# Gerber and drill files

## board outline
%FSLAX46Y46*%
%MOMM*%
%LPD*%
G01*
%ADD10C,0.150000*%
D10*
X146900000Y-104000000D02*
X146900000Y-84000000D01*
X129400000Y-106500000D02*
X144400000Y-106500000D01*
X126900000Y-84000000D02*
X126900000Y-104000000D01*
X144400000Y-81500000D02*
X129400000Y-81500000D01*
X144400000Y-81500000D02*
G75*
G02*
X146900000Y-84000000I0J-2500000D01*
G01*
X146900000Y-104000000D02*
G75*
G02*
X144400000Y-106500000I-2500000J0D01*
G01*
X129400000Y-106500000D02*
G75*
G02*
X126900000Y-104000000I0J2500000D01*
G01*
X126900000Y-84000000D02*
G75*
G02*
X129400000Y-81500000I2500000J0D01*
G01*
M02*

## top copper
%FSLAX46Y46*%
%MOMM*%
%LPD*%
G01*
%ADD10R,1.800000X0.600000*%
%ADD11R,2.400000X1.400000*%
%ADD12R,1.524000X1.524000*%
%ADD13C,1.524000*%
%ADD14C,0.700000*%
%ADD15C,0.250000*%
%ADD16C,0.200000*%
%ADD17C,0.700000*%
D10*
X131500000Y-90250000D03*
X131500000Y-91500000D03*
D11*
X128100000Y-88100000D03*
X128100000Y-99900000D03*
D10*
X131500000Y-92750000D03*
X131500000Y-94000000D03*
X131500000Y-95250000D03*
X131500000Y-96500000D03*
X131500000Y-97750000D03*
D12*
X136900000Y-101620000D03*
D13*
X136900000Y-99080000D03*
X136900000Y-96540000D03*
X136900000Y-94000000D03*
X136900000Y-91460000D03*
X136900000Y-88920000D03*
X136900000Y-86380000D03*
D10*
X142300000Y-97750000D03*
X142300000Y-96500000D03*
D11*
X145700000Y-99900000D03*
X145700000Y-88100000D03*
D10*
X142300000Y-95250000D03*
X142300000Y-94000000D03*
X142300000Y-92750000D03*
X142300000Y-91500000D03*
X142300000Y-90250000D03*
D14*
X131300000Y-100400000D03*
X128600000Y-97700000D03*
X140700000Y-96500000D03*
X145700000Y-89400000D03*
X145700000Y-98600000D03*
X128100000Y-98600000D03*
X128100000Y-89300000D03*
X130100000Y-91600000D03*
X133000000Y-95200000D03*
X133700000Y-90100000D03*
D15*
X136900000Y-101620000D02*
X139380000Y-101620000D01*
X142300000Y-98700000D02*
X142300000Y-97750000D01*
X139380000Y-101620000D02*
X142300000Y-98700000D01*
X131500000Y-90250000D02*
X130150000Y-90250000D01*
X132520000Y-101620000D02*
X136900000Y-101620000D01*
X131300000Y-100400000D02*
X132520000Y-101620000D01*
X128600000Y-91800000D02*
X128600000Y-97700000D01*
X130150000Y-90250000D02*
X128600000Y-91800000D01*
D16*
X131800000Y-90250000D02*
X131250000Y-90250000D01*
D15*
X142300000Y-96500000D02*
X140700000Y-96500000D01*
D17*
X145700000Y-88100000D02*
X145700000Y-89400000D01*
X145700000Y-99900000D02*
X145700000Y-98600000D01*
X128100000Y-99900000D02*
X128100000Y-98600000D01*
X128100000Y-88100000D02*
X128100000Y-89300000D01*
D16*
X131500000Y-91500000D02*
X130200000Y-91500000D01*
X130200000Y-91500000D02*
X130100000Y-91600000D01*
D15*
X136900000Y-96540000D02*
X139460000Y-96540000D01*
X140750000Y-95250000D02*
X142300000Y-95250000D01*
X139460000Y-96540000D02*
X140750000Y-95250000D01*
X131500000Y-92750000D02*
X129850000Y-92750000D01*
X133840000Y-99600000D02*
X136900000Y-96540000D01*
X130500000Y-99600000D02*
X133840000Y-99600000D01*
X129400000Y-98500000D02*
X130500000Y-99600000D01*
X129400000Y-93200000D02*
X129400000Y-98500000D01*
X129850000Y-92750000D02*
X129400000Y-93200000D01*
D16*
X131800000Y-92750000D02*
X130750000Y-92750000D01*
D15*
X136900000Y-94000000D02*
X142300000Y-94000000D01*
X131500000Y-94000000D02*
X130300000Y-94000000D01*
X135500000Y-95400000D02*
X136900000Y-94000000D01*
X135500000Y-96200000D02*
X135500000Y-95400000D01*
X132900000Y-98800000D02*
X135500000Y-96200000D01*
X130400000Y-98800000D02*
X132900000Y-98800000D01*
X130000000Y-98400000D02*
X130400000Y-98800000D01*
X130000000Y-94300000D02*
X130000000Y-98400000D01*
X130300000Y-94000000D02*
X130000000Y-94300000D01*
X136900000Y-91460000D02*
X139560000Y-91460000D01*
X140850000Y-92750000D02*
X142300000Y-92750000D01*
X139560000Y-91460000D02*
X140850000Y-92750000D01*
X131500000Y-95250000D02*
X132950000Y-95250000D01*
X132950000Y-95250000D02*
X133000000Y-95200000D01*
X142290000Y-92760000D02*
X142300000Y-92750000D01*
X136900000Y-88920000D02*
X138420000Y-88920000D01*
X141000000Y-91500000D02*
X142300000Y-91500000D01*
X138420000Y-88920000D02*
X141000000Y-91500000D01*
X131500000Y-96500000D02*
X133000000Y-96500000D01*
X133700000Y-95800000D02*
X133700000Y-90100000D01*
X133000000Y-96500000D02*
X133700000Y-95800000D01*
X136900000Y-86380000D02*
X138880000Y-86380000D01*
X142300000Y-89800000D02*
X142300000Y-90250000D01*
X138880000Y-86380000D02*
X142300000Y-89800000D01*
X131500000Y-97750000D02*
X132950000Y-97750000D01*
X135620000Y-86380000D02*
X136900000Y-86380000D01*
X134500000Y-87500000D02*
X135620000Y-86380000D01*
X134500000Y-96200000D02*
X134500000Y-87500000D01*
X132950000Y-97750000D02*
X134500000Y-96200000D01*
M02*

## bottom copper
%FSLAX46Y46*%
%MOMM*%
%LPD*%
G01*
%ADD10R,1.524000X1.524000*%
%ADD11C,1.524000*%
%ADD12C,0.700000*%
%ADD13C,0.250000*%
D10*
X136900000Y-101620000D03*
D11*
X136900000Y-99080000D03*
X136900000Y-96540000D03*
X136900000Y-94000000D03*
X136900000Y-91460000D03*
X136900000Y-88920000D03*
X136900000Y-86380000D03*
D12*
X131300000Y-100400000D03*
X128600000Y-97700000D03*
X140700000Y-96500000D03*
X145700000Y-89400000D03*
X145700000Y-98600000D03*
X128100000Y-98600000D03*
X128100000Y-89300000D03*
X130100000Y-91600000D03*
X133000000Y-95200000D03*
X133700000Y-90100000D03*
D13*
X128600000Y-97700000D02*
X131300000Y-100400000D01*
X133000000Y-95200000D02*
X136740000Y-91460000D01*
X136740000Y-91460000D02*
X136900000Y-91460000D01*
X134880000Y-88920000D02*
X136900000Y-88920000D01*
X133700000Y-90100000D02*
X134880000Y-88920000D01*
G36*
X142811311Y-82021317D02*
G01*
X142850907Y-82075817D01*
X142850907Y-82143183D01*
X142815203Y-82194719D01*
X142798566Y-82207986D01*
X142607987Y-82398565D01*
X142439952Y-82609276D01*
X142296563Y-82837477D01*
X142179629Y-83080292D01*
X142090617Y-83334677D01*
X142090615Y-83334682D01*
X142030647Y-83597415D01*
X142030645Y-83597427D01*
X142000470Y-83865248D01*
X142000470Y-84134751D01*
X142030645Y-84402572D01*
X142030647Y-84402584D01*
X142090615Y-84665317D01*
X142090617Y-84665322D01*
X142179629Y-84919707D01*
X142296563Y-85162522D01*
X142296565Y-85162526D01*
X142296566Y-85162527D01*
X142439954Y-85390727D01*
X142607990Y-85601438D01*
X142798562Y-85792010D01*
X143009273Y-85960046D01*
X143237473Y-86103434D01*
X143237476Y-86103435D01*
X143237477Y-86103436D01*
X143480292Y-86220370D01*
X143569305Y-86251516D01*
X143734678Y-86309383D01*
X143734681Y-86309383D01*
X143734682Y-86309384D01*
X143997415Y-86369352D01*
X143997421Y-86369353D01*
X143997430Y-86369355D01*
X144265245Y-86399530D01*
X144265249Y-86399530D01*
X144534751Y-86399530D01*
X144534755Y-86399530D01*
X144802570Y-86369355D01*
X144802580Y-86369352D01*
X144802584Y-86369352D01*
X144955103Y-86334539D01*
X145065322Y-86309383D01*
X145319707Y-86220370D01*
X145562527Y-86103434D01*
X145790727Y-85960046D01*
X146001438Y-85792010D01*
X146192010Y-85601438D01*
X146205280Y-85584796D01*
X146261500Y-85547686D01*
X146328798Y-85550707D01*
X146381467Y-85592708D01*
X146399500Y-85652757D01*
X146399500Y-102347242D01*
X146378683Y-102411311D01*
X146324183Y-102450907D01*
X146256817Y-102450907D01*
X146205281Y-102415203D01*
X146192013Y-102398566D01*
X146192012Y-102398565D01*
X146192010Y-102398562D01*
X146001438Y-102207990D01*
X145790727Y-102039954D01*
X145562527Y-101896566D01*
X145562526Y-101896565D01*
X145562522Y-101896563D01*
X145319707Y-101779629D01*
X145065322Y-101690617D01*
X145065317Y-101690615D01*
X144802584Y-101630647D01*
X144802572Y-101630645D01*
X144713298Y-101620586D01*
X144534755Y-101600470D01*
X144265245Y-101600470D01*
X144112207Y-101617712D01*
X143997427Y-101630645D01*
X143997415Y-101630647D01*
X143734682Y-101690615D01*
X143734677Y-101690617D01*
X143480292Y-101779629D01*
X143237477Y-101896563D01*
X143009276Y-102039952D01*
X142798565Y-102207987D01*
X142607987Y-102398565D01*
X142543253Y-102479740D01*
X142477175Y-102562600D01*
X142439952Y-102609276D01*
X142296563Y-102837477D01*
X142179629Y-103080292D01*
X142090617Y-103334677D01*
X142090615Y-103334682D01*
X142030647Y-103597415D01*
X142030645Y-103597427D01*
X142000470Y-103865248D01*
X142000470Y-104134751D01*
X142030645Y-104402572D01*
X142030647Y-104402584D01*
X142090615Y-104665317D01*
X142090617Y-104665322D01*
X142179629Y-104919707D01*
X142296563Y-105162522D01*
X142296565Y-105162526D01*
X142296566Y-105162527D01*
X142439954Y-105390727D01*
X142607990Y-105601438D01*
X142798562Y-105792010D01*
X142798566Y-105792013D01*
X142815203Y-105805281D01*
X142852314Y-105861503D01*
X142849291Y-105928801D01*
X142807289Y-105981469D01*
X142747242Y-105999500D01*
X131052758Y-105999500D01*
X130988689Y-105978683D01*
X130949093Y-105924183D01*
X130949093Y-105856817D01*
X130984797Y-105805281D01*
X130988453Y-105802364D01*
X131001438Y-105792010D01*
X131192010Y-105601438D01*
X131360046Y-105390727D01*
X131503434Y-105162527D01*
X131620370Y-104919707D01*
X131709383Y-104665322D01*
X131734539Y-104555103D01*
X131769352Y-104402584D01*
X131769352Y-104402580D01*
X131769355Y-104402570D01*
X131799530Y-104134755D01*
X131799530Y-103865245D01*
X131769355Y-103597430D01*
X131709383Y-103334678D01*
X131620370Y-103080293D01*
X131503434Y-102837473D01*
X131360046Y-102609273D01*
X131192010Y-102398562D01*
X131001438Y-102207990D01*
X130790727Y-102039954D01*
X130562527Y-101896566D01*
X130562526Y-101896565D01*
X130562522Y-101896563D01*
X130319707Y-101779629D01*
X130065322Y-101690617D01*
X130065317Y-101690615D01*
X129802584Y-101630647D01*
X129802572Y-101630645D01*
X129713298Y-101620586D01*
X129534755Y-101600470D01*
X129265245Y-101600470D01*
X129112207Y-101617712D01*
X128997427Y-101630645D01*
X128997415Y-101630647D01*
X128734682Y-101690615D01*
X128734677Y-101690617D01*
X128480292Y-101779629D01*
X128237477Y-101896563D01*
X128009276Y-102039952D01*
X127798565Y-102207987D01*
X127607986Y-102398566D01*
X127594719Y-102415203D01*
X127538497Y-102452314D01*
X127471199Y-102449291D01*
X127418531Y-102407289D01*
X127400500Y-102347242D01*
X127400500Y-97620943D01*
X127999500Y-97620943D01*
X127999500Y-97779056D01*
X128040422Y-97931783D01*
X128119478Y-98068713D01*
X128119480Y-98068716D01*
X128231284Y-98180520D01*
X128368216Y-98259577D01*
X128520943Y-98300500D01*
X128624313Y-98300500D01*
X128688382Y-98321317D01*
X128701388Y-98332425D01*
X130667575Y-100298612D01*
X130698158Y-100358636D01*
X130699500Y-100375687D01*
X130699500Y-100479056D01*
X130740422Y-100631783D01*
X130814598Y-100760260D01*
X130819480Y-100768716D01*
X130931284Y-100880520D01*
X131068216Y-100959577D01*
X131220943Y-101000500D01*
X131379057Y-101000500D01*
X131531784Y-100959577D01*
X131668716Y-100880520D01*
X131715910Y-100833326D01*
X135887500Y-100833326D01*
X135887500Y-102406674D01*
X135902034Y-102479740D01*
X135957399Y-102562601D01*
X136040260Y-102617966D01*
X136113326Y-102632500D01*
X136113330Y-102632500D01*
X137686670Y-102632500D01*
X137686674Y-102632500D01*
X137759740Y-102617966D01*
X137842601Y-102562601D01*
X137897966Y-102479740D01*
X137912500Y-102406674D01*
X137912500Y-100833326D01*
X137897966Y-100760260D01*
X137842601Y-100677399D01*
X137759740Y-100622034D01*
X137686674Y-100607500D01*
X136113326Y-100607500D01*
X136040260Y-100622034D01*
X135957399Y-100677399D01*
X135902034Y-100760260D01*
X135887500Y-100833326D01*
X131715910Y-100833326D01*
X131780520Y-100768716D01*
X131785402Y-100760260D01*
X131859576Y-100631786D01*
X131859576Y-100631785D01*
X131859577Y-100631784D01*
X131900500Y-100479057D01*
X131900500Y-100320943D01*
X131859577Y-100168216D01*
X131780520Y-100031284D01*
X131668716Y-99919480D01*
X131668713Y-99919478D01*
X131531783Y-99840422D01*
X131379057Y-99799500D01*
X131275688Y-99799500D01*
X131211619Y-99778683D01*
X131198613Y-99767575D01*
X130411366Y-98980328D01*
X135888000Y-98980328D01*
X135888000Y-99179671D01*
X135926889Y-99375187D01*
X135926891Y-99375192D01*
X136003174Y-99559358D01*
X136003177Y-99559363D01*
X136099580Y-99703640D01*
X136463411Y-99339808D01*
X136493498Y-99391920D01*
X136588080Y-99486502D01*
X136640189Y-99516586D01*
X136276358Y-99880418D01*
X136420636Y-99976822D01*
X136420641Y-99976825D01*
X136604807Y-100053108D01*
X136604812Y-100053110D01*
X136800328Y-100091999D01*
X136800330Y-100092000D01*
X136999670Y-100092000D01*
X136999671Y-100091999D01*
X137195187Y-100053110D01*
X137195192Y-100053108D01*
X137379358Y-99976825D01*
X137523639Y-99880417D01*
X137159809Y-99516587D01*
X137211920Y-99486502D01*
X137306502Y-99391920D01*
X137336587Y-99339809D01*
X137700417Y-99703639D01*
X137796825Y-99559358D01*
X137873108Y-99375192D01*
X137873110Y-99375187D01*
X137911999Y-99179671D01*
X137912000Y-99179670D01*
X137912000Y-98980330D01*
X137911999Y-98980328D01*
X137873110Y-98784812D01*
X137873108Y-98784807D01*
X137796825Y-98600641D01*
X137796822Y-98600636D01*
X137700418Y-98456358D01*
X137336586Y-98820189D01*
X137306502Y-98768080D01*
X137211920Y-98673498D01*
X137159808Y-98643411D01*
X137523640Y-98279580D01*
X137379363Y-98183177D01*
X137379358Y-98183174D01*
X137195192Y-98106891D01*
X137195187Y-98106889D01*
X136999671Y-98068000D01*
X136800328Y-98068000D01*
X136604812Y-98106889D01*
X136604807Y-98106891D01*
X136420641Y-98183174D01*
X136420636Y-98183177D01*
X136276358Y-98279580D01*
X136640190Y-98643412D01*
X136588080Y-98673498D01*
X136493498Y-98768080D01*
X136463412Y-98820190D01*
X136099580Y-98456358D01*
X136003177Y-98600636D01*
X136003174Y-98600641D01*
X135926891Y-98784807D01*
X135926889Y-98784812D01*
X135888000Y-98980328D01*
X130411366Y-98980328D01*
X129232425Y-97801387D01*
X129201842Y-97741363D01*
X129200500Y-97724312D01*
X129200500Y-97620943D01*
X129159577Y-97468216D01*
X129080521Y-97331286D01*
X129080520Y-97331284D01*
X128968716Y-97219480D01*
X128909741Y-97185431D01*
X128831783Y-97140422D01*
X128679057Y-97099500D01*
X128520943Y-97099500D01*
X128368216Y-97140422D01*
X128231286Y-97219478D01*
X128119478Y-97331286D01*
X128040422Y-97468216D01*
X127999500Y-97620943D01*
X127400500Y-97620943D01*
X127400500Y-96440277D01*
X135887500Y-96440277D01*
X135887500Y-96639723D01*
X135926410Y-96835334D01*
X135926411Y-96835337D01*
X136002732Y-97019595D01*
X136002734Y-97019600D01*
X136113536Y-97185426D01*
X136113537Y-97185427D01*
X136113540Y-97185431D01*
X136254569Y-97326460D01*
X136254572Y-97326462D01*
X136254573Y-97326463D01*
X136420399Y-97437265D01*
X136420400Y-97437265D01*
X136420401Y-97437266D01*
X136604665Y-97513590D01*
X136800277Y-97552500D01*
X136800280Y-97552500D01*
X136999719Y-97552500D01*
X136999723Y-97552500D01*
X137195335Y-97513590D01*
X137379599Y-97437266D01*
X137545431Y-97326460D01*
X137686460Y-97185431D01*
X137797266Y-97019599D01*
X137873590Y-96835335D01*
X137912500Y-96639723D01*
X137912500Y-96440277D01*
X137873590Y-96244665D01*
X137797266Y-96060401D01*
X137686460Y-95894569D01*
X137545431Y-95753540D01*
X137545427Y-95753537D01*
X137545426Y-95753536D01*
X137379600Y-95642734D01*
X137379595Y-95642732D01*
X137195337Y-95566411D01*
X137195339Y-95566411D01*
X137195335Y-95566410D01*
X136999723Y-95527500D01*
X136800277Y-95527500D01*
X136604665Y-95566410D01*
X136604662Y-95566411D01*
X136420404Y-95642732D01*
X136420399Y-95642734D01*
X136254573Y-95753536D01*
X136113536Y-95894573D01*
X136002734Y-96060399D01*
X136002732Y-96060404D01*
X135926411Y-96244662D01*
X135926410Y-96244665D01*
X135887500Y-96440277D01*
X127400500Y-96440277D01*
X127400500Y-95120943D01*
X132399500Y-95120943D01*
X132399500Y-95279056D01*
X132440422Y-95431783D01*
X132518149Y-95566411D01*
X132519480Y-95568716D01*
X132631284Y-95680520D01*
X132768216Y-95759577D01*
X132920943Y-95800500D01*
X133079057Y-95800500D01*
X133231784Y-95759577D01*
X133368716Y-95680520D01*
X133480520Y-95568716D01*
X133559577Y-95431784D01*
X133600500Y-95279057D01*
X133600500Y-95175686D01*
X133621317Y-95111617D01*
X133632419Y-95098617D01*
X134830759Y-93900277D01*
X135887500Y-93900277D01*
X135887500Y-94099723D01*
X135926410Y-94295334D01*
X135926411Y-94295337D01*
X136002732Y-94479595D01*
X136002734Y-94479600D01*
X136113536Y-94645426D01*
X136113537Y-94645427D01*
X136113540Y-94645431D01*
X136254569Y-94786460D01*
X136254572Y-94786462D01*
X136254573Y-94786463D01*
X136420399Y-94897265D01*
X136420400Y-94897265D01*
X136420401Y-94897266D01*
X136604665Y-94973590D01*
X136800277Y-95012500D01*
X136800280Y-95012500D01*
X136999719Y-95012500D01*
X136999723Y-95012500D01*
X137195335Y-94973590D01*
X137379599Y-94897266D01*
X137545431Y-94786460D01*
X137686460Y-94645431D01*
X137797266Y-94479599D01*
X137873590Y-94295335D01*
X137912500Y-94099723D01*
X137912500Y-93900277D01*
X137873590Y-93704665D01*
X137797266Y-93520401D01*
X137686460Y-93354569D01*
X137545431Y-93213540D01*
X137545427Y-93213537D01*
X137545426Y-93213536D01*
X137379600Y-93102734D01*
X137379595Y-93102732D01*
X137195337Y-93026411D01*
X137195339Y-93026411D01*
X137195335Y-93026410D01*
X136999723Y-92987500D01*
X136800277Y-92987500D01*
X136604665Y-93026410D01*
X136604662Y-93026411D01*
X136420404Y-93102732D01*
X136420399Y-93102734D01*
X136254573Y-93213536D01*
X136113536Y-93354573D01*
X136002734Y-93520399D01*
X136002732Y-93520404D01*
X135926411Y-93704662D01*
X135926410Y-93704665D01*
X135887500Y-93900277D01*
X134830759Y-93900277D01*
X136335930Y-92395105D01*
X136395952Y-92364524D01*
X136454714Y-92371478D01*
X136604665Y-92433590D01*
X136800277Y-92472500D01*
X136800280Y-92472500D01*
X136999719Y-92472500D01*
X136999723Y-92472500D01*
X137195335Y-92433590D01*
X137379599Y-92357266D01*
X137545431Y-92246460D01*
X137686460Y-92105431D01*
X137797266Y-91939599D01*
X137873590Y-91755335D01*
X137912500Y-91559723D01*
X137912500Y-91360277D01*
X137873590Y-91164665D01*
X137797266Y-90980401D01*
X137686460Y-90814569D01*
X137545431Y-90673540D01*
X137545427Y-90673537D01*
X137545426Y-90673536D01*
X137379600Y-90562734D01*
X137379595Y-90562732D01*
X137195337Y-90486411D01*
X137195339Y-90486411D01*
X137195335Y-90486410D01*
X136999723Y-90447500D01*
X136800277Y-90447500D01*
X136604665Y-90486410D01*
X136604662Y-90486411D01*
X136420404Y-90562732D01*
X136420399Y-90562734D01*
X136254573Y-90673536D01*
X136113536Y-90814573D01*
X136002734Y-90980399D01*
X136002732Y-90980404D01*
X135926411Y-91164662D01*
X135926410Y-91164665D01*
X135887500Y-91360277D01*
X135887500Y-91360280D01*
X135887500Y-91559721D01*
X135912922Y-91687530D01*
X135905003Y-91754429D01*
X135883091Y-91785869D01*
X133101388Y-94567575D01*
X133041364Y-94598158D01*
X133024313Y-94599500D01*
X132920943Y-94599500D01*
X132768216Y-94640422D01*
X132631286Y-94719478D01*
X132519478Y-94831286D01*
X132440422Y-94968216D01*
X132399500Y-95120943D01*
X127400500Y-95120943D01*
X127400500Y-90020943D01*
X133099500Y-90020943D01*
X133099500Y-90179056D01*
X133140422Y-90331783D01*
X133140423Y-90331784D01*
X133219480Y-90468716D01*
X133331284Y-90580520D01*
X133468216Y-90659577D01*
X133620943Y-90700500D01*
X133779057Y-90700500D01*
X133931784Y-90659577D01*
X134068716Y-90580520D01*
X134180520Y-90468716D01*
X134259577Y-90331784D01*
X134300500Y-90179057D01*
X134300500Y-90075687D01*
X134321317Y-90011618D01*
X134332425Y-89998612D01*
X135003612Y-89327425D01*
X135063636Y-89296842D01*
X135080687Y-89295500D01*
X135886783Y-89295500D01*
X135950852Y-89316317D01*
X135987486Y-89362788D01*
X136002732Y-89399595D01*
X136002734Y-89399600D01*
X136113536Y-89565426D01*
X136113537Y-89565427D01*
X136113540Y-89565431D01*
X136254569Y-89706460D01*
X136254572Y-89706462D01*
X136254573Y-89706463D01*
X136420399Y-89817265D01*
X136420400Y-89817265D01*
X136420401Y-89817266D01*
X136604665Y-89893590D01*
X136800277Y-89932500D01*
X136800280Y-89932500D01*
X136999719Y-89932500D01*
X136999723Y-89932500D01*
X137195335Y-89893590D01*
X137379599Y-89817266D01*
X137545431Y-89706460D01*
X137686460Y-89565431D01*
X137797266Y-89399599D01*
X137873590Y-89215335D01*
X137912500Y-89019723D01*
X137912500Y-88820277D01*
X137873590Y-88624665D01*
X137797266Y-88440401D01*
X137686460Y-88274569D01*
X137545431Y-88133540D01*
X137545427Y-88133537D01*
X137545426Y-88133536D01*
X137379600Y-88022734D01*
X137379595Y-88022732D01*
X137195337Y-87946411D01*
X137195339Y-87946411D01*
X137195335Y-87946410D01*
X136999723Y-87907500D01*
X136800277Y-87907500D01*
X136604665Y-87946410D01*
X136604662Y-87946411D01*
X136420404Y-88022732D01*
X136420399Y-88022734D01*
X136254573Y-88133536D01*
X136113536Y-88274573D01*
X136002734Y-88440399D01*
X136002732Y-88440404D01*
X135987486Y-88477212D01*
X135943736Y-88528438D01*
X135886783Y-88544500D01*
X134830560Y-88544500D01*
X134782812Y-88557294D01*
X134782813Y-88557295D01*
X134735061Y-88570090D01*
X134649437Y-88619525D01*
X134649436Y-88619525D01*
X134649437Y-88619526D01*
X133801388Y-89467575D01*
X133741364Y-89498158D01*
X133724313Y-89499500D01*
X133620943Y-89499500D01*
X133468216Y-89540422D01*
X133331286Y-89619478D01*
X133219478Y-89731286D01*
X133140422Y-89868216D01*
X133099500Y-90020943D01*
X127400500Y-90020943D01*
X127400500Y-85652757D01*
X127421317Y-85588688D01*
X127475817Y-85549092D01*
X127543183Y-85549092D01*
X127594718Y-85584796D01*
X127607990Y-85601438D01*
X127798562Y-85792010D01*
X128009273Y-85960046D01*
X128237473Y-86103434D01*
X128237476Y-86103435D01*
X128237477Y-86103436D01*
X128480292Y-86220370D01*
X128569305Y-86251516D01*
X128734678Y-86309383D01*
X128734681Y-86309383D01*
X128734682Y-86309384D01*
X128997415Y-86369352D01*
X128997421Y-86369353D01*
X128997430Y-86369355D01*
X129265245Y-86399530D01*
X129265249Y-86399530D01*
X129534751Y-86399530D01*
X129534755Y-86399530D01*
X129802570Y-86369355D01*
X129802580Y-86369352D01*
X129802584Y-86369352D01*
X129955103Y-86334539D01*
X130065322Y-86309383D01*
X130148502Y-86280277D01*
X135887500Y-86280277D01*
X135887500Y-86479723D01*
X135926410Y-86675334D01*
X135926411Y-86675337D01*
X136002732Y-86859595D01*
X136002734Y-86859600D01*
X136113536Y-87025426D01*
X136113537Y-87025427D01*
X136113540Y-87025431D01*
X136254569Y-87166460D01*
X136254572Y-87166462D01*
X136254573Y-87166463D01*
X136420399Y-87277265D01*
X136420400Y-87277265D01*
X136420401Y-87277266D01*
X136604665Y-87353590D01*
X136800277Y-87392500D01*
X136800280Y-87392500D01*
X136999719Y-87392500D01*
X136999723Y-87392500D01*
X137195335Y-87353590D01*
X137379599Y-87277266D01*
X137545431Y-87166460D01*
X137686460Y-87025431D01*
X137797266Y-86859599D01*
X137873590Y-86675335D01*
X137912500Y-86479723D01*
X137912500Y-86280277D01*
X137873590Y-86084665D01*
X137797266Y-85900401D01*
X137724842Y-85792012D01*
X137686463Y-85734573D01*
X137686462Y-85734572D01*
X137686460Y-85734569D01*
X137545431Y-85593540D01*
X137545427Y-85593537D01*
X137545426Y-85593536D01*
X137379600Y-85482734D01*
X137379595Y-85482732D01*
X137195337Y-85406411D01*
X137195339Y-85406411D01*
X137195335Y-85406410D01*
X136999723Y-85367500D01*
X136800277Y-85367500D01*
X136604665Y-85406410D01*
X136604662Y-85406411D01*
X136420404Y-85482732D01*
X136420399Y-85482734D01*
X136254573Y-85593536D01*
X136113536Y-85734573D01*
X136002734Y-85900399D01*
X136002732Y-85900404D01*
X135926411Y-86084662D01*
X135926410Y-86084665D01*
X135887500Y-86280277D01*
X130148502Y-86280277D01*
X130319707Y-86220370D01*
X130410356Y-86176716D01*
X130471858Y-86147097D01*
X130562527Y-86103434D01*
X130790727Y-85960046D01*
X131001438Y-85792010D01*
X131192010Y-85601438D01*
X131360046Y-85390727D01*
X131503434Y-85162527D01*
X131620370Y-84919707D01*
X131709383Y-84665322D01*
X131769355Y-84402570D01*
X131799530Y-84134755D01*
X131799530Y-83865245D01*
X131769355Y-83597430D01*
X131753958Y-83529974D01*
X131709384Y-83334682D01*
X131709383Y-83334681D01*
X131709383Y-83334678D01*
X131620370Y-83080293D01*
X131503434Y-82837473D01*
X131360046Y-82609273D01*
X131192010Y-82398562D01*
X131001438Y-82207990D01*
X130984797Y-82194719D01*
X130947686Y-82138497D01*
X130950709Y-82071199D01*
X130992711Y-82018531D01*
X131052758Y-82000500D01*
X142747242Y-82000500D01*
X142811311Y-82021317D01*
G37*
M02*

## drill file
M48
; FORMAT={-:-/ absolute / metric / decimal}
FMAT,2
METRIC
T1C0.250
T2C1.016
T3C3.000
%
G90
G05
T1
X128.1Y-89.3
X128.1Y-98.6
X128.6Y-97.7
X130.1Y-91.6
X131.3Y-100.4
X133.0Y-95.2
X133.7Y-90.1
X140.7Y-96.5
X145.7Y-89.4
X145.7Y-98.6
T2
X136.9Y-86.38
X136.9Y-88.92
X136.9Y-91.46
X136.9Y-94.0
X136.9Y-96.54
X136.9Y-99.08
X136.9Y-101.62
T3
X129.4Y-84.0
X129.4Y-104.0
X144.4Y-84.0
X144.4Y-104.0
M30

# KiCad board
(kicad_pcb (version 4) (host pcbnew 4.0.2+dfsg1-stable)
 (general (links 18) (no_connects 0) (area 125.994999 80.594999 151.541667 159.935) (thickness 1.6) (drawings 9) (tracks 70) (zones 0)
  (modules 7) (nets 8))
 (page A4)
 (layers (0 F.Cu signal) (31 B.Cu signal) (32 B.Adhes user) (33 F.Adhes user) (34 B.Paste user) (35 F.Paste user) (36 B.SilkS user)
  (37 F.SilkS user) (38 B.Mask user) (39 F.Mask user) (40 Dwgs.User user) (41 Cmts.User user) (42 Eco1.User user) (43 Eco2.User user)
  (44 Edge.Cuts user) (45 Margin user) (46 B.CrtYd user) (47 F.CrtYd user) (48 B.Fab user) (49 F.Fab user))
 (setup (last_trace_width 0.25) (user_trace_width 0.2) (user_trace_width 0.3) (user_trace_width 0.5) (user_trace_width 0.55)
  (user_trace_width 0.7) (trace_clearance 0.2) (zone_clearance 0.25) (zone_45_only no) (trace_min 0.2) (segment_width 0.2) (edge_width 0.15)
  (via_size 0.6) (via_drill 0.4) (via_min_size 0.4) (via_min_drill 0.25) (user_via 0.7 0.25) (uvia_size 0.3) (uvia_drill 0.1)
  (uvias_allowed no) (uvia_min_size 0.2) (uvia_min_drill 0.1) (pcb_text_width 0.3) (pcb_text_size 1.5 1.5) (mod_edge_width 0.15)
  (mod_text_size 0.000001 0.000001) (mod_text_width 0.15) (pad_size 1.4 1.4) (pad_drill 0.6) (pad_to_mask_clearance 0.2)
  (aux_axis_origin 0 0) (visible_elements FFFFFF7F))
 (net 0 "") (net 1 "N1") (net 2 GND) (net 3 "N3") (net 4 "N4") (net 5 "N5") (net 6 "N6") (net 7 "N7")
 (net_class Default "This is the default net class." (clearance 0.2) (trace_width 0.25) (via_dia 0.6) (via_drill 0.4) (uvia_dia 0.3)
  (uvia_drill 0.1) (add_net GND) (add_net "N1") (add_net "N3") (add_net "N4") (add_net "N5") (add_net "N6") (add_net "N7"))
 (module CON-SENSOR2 (layer F.Cu) (at 126.9 94 270)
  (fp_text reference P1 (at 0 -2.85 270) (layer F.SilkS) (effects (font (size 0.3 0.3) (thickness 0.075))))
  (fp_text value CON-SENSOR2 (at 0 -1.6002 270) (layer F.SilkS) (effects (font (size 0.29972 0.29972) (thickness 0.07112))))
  (pad 1 smd rect (at -3.75 -4.6 270) (size 0.6 1.8) (layers F.Cu F.Paste F.Mask) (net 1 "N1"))
  (pad 2 smd rect (at -2.5 -4.6 270) (size 0.6 1.8) (layers F.Cu F.Paste F.Mask) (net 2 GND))
  (pad EP smd rect (at -5.9 -1.2 270) (size 1.4 2.4) (layers F.Cu F.Paste F.Mask) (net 2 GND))
  (pad EP smd rect (at 5.9 -1.2 270) (size 1.4 2.4) (layers F.Cu F.Paste F.Mask) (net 2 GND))
  (pad 3 smd rect (at -1.25 -4.6 270) (size 0.6 1.8) (layers F.Cu F.Paste F.Mask) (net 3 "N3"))
  (pad 4 smd rect (at 0 -4.6 270) (size 0.6 1.8) (layers F.Cu F.Paste F.Mask) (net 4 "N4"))
  (pad 5 smd rect (at 1.25 -4.6 270) (size 0.6 1.8) (layers F.Cu F.Paste F.Mask) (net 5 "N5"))
  (pad 6 smd rect (at 2.5 -4.6 270) (size 0.6 1.8) (layers F.Cu F.Paste F.Mask) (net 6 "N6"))
  (pad 7 smd rect (at 3.75 -4.6 270) (size 0.6 1.8) (layers F.Cu F.Paste F.Mask) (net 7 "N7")))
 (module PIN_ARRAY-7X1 (layer F.Cu) (at 136.9 94 90)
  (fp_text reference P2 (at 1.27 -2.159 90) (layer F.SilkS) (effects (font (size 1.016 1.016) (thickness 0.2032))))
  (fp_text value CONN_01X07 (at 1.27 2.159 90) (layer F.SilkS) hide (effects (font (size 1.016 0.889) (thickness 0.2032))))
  (pad 1 thru_hole rect (at -7.62 0 90) (size 1.524 1.524) (drill 1.016) (layers *.Cu *.Mask F.SilkS) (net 1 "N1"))
  (pad 2 thru_hole circle (at -5.08 0 90) (size 1.524 1.524) (drill 1.016) (layers *.Cu *.Mask F.SilkS) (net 2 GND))
  (pad 3 thru_hole circle (at -2.54 0 90) (size 1.524 1.524) (drill 1.016) (layers *.Cu *.Mask F.SilkS) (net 3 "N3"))
  (pad 4 thru_hole circle (at 0 0 90) (size 1.524 1.524) (drill 1.016) (layers *.Cu *.Mask F.SilkS) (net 4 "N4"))
  (pad 5 thru_hole circle (at 2.54 0 90) (size 1.524 1.524) (drill 1.016) (layers *.Cu *.Mask F.SilkS) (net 5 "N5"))
  (pad 6 thru_hole circle (at 5.08 0 90) (size 1.524 1.524) (drill 1.016) (layers *.Cu *.Mask F.SilkS) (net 6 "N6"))
  (pad 7 thru_hole circle (at 7.62 0 90) (size 1.524 1.524) (drill 1.016) (layers *.Cu *.Mask F.SilkS) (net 7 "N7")))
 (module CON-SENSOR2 (layer F.Cu) (at 146.9 94 90)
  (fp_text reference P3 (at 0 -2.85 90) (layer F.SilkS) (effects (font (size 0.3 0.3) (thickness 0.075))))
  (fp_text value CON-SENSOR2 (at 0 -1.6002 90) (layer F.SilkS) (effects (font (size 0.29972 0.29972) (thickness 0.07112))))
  (pad 1 smd rect (at -3.75 -4.6 90) (size 0.6 1.8) (layers F.Cu F.Paste F.Mask) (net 1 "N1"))
  (pad 2 smd rect (at -2.5 -4.6 90) (size 0.6 1.8) (layers F.Cu F.Paste F.Mask) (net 2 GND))
  (pad EP smd rect (at -5.9 -1.2 90) (size 1.4 2.4) (layers F.Cu F.Paste F.Mask) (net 2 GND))
  (pad EP smd rect (at 5.9 -1.2 90) (size 1.4 2.4) (layers F.Cu F.Paste F.Mask) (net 2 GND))
  (pad 3 smd rect (at -1.25 -4.6 90) (size 0.6 1.8) (layers F.Cu F.Paste F.Mask) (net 3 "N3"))
  (pad 4 smd rect (at 0 -4.6 90) (size 0.6 1.8) (layers F.Cu F.Paste F.Mask) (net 4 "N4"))
  (pad 5 smd rect (at 1.25 -4.6 90) (size 0.6 1.8) (layers F.Cu F.Paste F.Mask) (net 5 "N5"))
  (pad 6 smd rect (at 2.5 -4.6 90) (size 0.6 1.8) (layers F.Cu F.Paste F.Mask) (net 6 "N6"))
  (pad 7 smd rect (at 3.75 -4.6 90) (size 0.6 1.8) (layers F.Cu F.Paste F.Mask) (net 7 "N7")))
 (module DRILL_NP (layer F.Cu) (at 129.4 84)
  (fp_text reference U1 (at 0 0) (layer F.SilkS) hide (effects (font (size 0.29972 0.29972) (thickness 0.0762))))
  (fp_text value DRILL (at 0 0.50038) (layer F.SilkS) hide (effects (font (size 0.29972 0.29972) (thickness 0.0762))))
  (pad "" np_thru_hole circle (at 0 0) (size 2.99974 2.99974) (drill 2.99974) (layers *.Cu *.Mask F.SilkS) (clearance 0.89916)))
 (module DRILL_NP (layer F.Cu) (at 144.4 84)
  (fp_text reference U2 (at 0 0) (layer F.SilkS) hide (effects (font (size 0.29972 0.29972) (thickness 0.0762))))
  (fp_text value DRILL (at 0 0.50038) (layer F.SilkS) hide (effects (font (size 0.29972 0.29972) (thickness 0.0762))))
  (pad "" np_thru_hole circle (at 0 0) (size 2.99974 2.99974) (drill 2.99974) (layers *.Cu *.Mask F.SilkS) (clearance 0.89916)))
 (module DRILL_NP (layer F.Cu) (at 129.4 104)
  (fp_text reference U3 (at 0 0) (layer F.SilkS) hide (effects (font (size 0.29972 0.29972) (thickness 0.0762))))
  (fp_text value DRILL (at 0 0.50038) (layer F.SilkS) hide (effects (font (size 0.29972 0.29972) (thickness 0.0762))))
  (pad "" np_thru_hole circle (at 0 0) (size 2.99974 2.99974) (drill 2.99974) (layers *.Cu *.Mask F.SilkS) (clearance 0.89916)))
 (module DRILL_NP (layer F.Cu) (at 144.4 104)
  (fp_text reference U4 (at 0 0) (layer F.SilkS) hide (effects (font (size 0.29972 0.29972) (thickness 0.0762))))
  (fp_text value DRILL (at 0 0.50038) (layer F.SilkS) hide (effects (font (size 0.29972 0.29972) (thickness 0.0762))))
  (pad "" np_thru_hole circle (at 0 0) (size 2.99974 2.99974) (drill 2.99974) (layers *.Cu *.Mask F.SilkS) (clearance 0.89916)))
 (gr_line (start 146.9 104) (end 146.9 84) (angle 90) (layer Edge.Cuts) (width 0.15))
 (gr_line (start 129.4 106.5) (end 144.4 106.5) (angle 90) (layer Edge.Cuts) (width 0.15))
 (gr_line (start 126.9 84) (end 126.9 104) (angle 90) (layer Edge.Cuts) (width 0.15))
 (gr_line (start 144.4 81.5) (end 129.4 81.5) (angle 90) (layer Edge.Cuts) (width 0.15))
 (gr_arc (start 144.4 84) (end 144.4 81.5) (angle 90) (layer Edge.Cuts) (width 0.15))
 (gr_arc (start 144.4 104) (end 146.9 104) (angle 90) (layer Edge.Cuts) (width 0.15))
 (gr_arc (start 129.4 104) (end 129.4 106.5) (angle 90) (layer Edge.Cuts) (width 0.15))
 (gr_arc (start 129.4 84) (end 126.9 84) (angle 90) (layer Edge.Cuts) (width 0.15))
 (segment (start 136.9 101.62) (end 139.38 101.62) (width 0.25) (layer F.Cu) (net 1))
 (segment (start 142.3 98.7) (end 142.3 97.75) (width 0.25) (layer F.Cu) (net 1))
 (segment (start 139.38 101.62) (end 142.3 98.7) (width 0.25) (layer F.Cu) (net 1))
 (segment (start 131.5 90.25) (end 130.15 90.25) (width 0.25) (layer F.Cu) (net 1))
 (segment (start 132.52 101.62) (end 136.9 101.62) (width 0.25) (layer F.Cu) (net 1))
 (segment (start 131.3 100.4) (end 132.52 101.62) (width 0.25) (layer F.Cu) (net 1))
 (via (at 131.3 100.4) (size 0.7) (drill 0.25) (layers F.Cu B.Cu) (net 1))
 (segment (start 128.6 97.7) (end 131.3 100.4) (width 0.25) (layer B.Cu) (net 1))
 (via (at 128.6 97.7) (size 0.7) (drill 0.25) (layers F.Cu B.Cu) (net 1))
 (segment (start 128.6 91.8) (end 128.6 97.7) (width 0.25) (layer F.Cu) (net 1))
 (segment (start 130.15 90.25) (end 128.6 91.8) (width 0.25) (layer F.Cu) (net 1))
 (segment (start 131.8 90.25) (end 131.25 90.25) (width 0.2) (layer F.Cu) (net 1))
 (segment (start 142.3 96.5) (end 140.7 96.5) (width 0.25) (layer F.Cu) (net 2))
 (via (at 140.7 96.5) (size 0.7) (drill 0.25) (layers F.Cu B.Cu) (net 2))
 (segment (start 145.7 88.1) (end 145.7 89.4) (width 0.7) (layer F.Cu) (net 2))
 (via (at 145.7 89.4) (size 0.7) (drill 0.25) (layers F.Cu B.Cu) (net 2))
 (segment (start 145.7 99.9) (end 145.7 98.6) (width 0.7) (layer F.Cu) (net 2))
 (via (at 145.7 98.6) (size 0.7) (drill 0.25) (layers F.Cu B.Cu) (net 2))
 (segment (start 128.1 99.9) (end 128.1 98.6) (width 0.7) (layer F.Cu) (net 2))
 (via (at 128.1 98.6) (size 0.7) (drill 0.25) (layers F.Cu B.Cu) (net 2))
 (segment (start 128.1 88.1) (end 128.1 89.3) (width 0.7) (layer F.Cu) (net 2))
 (via (at 128.1 89.3) (size 0.7) (drill 0.25) (layers F.Cu B.Cu) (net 2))
 (segment (start 131.5 91.5) (end 130.2 91.5) (width 0.2) (layer F.Cu) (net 2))
 (via (at 130.1 91.6) (size 0.7) (drill 0.25) (layers F.Cu B.Cu) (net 2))
 (segment (start 130.2 91.5) (end 130.1 91.6) (width 0.2) (layer F.Cu) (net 2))
 (segment (start 136.9 96.54) (end 139.46 96.54) (width 0.25) (layer F.Cu) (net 3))
 (segment (start 140.75 95.25) (end 142.3 95.25) (width 0.25) (layer F.Cu) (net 3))
 (segment (start 139.46 96.54) (end 140.75 95.25) (width 0.25) (layer F.Cu) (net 3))
 (segment (start 131.5 92.75) (end 129.85 92.75) (width 0.25) (layer F.Cu) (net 3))
 (segment (start 133.84 99.6) (end 136.9 96.54) (width 0.25) (layer F.Cu) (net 3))
 (segment (start 130.5 99.6) (end 133.84 99.6) (width 0.25) (layer F.Cu) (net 3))
 (segment (start 129.4 98.5) (end 130.5 99.6) (width 0.25) (layer F.Cu) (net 3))
 (segment (start 129.4 93.2) (end 129.4 98.5) (width 0.25) (layer F.Cu) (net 3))
 (segment (start 129.85 92.75) (end 129.4 93.2) (width 0.25) (layer F.Cu) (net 3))
 (segment (start 131.8 92.75) (end 130.75 92.75) (width 0.2) (layer F.Cu) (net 3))
 (segment (start 136.9 94) (end 142.3 94) (width 0.25) (layer F.Cu) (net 4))
 (segment (start 131.5 94) (end 130.3 94) (width 0.25) (layer F.Cu) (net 4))
 (segment (start 135.5 95.4) (end 136.9 94) (width 0.25) (layer F.Cu) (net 4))
 (segment (start 135.5 96.2) (end 135.5 95.4) (width 0.25) (layer F.Cu) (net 4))
 (segment (start 132.9 98.8) (end 135.5 96.2) (width 0.25) (layer F.Cu) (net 4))
 (segment (start 130.4 98.8) (end 132.9 98.8) (width 0.25) (layer F.Cu) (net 4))
 (segment (start 130 98.4) (end 130.4 98.8) (width 0.25) (layer F.Cu) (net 4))
 (segment (start 130 94.3) (end 130 98.4) (width 0.25) (layer F.Cu) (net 4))
 (segment (start 130.3 94) (end 130 94.3) (width 0.25) (layer F.Cu) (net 4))
 (segment (start 136.9 91.46) (end 139.56 91.46) (width 0.25) (layer F.Cu) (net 5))
 (segment (start 140.85 92.75) (end 142.3 92.75) (width 0.25) (layer F.Cu) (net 5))
 (segment (start 139.56 91.46) (end 140.85 92.75) (width 0.25) (layer F.Cu) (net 5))
 (segment (start 131.5 95.25) (end 132.95 95.25) (width 0.25) (layer F.Cu) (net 5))
 (segment (start 133 95.2) (end 136.74 91.46) (width 0.25) (layer B.Cu) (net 5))
 (via (at 133 95.2) (size 0.7) (drill 0.25) (layers F.Cu B.Cu) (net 5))
 (segment (start 132.95 95.25) (end 133 95.2) (width 0.25) (layer F.Cu) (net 5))
 (segment (start 136.74 91.46) (end 136.9 91.46) (width 0.25) (layer B.Cu) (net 5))
 (segment (start 142.29 92.76) (end 142.3 92.75) (width 0.25) (layer F.Cu) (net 5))
 (segment (start 136.9 88.92) (end 138.42 88.92) (width 0.25) (layer F.Cu) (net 6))
 (segment (start 141 91.5) (end 142.3 91.5) (width 0.25) (layer F.Cu) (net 6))
 (segment (start 138.42 88.92) (end 141 91.5) (width 0.25) (layer F.Cu) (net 6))
 (segment (start 131.5 96.5) (end 133 96.5) (width 0.25) (layer F.Cu) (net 6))
 (segment (start 134.88 88.92) (end 136.9 88.92) (width 0.25) (layer B.Cu) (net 6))
 (segment (start 133.7 90.1) (end 134.88 88.92) (width 0.25) (layer B.Cu) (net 6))
 (via (at 133.7 90.1) (size 0.7) (drill 0.25) (layers F.Cu B.Cu) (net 6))
 (segment (start 133.7 95.8) (end 133.7 90.1) (width 0.25) (layer F.Cu) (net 6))
 (segment (start 133 96.5) (end 133.7 95.8) (width 0.25) (layer F.Cu) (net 6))
 (segment (start 136.9 86.38) (end 138.88 86.38) (width 0.25) (layer F.Cu) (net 7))
 (segment (start 142.3 89.8) (end 142.3 90.25) (width 0.25) (layer F.Cu) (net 7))
 (segment (start 138.88 86.38) (end 142.3 89.8) (width 0.25) (layer F.Cu) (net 7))
 (segment (start 131.5 97.75) (end 132.95 97.75) (width 0.25) (layer F.Cu) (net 7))
 (segment (start 135.62 86.38) (end 136.9 86.38) (width 0.25) (layer F.Cu) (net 7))
 (segment (start 134.5 87.5) (end 135.62 86.38) (width 0.25) (layer F.Cu) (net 7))
 (segment (start 134.5 96.2) (end 134.5 87.5) (width 0.25) (layer F.Cu) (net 7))
 (segment (start 132.95 97.75) (end 134.5 96.2) (width 0.25) (layer F.Cu) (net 7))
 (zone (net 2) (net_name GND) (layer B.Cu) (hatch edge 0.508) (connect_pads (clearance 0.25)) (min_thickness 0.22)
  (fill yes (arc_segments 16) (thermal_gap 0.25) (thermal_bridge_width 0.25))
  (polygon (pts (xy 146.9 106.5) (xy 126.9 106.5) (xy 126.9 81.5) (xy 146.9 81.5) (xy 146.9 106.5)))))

